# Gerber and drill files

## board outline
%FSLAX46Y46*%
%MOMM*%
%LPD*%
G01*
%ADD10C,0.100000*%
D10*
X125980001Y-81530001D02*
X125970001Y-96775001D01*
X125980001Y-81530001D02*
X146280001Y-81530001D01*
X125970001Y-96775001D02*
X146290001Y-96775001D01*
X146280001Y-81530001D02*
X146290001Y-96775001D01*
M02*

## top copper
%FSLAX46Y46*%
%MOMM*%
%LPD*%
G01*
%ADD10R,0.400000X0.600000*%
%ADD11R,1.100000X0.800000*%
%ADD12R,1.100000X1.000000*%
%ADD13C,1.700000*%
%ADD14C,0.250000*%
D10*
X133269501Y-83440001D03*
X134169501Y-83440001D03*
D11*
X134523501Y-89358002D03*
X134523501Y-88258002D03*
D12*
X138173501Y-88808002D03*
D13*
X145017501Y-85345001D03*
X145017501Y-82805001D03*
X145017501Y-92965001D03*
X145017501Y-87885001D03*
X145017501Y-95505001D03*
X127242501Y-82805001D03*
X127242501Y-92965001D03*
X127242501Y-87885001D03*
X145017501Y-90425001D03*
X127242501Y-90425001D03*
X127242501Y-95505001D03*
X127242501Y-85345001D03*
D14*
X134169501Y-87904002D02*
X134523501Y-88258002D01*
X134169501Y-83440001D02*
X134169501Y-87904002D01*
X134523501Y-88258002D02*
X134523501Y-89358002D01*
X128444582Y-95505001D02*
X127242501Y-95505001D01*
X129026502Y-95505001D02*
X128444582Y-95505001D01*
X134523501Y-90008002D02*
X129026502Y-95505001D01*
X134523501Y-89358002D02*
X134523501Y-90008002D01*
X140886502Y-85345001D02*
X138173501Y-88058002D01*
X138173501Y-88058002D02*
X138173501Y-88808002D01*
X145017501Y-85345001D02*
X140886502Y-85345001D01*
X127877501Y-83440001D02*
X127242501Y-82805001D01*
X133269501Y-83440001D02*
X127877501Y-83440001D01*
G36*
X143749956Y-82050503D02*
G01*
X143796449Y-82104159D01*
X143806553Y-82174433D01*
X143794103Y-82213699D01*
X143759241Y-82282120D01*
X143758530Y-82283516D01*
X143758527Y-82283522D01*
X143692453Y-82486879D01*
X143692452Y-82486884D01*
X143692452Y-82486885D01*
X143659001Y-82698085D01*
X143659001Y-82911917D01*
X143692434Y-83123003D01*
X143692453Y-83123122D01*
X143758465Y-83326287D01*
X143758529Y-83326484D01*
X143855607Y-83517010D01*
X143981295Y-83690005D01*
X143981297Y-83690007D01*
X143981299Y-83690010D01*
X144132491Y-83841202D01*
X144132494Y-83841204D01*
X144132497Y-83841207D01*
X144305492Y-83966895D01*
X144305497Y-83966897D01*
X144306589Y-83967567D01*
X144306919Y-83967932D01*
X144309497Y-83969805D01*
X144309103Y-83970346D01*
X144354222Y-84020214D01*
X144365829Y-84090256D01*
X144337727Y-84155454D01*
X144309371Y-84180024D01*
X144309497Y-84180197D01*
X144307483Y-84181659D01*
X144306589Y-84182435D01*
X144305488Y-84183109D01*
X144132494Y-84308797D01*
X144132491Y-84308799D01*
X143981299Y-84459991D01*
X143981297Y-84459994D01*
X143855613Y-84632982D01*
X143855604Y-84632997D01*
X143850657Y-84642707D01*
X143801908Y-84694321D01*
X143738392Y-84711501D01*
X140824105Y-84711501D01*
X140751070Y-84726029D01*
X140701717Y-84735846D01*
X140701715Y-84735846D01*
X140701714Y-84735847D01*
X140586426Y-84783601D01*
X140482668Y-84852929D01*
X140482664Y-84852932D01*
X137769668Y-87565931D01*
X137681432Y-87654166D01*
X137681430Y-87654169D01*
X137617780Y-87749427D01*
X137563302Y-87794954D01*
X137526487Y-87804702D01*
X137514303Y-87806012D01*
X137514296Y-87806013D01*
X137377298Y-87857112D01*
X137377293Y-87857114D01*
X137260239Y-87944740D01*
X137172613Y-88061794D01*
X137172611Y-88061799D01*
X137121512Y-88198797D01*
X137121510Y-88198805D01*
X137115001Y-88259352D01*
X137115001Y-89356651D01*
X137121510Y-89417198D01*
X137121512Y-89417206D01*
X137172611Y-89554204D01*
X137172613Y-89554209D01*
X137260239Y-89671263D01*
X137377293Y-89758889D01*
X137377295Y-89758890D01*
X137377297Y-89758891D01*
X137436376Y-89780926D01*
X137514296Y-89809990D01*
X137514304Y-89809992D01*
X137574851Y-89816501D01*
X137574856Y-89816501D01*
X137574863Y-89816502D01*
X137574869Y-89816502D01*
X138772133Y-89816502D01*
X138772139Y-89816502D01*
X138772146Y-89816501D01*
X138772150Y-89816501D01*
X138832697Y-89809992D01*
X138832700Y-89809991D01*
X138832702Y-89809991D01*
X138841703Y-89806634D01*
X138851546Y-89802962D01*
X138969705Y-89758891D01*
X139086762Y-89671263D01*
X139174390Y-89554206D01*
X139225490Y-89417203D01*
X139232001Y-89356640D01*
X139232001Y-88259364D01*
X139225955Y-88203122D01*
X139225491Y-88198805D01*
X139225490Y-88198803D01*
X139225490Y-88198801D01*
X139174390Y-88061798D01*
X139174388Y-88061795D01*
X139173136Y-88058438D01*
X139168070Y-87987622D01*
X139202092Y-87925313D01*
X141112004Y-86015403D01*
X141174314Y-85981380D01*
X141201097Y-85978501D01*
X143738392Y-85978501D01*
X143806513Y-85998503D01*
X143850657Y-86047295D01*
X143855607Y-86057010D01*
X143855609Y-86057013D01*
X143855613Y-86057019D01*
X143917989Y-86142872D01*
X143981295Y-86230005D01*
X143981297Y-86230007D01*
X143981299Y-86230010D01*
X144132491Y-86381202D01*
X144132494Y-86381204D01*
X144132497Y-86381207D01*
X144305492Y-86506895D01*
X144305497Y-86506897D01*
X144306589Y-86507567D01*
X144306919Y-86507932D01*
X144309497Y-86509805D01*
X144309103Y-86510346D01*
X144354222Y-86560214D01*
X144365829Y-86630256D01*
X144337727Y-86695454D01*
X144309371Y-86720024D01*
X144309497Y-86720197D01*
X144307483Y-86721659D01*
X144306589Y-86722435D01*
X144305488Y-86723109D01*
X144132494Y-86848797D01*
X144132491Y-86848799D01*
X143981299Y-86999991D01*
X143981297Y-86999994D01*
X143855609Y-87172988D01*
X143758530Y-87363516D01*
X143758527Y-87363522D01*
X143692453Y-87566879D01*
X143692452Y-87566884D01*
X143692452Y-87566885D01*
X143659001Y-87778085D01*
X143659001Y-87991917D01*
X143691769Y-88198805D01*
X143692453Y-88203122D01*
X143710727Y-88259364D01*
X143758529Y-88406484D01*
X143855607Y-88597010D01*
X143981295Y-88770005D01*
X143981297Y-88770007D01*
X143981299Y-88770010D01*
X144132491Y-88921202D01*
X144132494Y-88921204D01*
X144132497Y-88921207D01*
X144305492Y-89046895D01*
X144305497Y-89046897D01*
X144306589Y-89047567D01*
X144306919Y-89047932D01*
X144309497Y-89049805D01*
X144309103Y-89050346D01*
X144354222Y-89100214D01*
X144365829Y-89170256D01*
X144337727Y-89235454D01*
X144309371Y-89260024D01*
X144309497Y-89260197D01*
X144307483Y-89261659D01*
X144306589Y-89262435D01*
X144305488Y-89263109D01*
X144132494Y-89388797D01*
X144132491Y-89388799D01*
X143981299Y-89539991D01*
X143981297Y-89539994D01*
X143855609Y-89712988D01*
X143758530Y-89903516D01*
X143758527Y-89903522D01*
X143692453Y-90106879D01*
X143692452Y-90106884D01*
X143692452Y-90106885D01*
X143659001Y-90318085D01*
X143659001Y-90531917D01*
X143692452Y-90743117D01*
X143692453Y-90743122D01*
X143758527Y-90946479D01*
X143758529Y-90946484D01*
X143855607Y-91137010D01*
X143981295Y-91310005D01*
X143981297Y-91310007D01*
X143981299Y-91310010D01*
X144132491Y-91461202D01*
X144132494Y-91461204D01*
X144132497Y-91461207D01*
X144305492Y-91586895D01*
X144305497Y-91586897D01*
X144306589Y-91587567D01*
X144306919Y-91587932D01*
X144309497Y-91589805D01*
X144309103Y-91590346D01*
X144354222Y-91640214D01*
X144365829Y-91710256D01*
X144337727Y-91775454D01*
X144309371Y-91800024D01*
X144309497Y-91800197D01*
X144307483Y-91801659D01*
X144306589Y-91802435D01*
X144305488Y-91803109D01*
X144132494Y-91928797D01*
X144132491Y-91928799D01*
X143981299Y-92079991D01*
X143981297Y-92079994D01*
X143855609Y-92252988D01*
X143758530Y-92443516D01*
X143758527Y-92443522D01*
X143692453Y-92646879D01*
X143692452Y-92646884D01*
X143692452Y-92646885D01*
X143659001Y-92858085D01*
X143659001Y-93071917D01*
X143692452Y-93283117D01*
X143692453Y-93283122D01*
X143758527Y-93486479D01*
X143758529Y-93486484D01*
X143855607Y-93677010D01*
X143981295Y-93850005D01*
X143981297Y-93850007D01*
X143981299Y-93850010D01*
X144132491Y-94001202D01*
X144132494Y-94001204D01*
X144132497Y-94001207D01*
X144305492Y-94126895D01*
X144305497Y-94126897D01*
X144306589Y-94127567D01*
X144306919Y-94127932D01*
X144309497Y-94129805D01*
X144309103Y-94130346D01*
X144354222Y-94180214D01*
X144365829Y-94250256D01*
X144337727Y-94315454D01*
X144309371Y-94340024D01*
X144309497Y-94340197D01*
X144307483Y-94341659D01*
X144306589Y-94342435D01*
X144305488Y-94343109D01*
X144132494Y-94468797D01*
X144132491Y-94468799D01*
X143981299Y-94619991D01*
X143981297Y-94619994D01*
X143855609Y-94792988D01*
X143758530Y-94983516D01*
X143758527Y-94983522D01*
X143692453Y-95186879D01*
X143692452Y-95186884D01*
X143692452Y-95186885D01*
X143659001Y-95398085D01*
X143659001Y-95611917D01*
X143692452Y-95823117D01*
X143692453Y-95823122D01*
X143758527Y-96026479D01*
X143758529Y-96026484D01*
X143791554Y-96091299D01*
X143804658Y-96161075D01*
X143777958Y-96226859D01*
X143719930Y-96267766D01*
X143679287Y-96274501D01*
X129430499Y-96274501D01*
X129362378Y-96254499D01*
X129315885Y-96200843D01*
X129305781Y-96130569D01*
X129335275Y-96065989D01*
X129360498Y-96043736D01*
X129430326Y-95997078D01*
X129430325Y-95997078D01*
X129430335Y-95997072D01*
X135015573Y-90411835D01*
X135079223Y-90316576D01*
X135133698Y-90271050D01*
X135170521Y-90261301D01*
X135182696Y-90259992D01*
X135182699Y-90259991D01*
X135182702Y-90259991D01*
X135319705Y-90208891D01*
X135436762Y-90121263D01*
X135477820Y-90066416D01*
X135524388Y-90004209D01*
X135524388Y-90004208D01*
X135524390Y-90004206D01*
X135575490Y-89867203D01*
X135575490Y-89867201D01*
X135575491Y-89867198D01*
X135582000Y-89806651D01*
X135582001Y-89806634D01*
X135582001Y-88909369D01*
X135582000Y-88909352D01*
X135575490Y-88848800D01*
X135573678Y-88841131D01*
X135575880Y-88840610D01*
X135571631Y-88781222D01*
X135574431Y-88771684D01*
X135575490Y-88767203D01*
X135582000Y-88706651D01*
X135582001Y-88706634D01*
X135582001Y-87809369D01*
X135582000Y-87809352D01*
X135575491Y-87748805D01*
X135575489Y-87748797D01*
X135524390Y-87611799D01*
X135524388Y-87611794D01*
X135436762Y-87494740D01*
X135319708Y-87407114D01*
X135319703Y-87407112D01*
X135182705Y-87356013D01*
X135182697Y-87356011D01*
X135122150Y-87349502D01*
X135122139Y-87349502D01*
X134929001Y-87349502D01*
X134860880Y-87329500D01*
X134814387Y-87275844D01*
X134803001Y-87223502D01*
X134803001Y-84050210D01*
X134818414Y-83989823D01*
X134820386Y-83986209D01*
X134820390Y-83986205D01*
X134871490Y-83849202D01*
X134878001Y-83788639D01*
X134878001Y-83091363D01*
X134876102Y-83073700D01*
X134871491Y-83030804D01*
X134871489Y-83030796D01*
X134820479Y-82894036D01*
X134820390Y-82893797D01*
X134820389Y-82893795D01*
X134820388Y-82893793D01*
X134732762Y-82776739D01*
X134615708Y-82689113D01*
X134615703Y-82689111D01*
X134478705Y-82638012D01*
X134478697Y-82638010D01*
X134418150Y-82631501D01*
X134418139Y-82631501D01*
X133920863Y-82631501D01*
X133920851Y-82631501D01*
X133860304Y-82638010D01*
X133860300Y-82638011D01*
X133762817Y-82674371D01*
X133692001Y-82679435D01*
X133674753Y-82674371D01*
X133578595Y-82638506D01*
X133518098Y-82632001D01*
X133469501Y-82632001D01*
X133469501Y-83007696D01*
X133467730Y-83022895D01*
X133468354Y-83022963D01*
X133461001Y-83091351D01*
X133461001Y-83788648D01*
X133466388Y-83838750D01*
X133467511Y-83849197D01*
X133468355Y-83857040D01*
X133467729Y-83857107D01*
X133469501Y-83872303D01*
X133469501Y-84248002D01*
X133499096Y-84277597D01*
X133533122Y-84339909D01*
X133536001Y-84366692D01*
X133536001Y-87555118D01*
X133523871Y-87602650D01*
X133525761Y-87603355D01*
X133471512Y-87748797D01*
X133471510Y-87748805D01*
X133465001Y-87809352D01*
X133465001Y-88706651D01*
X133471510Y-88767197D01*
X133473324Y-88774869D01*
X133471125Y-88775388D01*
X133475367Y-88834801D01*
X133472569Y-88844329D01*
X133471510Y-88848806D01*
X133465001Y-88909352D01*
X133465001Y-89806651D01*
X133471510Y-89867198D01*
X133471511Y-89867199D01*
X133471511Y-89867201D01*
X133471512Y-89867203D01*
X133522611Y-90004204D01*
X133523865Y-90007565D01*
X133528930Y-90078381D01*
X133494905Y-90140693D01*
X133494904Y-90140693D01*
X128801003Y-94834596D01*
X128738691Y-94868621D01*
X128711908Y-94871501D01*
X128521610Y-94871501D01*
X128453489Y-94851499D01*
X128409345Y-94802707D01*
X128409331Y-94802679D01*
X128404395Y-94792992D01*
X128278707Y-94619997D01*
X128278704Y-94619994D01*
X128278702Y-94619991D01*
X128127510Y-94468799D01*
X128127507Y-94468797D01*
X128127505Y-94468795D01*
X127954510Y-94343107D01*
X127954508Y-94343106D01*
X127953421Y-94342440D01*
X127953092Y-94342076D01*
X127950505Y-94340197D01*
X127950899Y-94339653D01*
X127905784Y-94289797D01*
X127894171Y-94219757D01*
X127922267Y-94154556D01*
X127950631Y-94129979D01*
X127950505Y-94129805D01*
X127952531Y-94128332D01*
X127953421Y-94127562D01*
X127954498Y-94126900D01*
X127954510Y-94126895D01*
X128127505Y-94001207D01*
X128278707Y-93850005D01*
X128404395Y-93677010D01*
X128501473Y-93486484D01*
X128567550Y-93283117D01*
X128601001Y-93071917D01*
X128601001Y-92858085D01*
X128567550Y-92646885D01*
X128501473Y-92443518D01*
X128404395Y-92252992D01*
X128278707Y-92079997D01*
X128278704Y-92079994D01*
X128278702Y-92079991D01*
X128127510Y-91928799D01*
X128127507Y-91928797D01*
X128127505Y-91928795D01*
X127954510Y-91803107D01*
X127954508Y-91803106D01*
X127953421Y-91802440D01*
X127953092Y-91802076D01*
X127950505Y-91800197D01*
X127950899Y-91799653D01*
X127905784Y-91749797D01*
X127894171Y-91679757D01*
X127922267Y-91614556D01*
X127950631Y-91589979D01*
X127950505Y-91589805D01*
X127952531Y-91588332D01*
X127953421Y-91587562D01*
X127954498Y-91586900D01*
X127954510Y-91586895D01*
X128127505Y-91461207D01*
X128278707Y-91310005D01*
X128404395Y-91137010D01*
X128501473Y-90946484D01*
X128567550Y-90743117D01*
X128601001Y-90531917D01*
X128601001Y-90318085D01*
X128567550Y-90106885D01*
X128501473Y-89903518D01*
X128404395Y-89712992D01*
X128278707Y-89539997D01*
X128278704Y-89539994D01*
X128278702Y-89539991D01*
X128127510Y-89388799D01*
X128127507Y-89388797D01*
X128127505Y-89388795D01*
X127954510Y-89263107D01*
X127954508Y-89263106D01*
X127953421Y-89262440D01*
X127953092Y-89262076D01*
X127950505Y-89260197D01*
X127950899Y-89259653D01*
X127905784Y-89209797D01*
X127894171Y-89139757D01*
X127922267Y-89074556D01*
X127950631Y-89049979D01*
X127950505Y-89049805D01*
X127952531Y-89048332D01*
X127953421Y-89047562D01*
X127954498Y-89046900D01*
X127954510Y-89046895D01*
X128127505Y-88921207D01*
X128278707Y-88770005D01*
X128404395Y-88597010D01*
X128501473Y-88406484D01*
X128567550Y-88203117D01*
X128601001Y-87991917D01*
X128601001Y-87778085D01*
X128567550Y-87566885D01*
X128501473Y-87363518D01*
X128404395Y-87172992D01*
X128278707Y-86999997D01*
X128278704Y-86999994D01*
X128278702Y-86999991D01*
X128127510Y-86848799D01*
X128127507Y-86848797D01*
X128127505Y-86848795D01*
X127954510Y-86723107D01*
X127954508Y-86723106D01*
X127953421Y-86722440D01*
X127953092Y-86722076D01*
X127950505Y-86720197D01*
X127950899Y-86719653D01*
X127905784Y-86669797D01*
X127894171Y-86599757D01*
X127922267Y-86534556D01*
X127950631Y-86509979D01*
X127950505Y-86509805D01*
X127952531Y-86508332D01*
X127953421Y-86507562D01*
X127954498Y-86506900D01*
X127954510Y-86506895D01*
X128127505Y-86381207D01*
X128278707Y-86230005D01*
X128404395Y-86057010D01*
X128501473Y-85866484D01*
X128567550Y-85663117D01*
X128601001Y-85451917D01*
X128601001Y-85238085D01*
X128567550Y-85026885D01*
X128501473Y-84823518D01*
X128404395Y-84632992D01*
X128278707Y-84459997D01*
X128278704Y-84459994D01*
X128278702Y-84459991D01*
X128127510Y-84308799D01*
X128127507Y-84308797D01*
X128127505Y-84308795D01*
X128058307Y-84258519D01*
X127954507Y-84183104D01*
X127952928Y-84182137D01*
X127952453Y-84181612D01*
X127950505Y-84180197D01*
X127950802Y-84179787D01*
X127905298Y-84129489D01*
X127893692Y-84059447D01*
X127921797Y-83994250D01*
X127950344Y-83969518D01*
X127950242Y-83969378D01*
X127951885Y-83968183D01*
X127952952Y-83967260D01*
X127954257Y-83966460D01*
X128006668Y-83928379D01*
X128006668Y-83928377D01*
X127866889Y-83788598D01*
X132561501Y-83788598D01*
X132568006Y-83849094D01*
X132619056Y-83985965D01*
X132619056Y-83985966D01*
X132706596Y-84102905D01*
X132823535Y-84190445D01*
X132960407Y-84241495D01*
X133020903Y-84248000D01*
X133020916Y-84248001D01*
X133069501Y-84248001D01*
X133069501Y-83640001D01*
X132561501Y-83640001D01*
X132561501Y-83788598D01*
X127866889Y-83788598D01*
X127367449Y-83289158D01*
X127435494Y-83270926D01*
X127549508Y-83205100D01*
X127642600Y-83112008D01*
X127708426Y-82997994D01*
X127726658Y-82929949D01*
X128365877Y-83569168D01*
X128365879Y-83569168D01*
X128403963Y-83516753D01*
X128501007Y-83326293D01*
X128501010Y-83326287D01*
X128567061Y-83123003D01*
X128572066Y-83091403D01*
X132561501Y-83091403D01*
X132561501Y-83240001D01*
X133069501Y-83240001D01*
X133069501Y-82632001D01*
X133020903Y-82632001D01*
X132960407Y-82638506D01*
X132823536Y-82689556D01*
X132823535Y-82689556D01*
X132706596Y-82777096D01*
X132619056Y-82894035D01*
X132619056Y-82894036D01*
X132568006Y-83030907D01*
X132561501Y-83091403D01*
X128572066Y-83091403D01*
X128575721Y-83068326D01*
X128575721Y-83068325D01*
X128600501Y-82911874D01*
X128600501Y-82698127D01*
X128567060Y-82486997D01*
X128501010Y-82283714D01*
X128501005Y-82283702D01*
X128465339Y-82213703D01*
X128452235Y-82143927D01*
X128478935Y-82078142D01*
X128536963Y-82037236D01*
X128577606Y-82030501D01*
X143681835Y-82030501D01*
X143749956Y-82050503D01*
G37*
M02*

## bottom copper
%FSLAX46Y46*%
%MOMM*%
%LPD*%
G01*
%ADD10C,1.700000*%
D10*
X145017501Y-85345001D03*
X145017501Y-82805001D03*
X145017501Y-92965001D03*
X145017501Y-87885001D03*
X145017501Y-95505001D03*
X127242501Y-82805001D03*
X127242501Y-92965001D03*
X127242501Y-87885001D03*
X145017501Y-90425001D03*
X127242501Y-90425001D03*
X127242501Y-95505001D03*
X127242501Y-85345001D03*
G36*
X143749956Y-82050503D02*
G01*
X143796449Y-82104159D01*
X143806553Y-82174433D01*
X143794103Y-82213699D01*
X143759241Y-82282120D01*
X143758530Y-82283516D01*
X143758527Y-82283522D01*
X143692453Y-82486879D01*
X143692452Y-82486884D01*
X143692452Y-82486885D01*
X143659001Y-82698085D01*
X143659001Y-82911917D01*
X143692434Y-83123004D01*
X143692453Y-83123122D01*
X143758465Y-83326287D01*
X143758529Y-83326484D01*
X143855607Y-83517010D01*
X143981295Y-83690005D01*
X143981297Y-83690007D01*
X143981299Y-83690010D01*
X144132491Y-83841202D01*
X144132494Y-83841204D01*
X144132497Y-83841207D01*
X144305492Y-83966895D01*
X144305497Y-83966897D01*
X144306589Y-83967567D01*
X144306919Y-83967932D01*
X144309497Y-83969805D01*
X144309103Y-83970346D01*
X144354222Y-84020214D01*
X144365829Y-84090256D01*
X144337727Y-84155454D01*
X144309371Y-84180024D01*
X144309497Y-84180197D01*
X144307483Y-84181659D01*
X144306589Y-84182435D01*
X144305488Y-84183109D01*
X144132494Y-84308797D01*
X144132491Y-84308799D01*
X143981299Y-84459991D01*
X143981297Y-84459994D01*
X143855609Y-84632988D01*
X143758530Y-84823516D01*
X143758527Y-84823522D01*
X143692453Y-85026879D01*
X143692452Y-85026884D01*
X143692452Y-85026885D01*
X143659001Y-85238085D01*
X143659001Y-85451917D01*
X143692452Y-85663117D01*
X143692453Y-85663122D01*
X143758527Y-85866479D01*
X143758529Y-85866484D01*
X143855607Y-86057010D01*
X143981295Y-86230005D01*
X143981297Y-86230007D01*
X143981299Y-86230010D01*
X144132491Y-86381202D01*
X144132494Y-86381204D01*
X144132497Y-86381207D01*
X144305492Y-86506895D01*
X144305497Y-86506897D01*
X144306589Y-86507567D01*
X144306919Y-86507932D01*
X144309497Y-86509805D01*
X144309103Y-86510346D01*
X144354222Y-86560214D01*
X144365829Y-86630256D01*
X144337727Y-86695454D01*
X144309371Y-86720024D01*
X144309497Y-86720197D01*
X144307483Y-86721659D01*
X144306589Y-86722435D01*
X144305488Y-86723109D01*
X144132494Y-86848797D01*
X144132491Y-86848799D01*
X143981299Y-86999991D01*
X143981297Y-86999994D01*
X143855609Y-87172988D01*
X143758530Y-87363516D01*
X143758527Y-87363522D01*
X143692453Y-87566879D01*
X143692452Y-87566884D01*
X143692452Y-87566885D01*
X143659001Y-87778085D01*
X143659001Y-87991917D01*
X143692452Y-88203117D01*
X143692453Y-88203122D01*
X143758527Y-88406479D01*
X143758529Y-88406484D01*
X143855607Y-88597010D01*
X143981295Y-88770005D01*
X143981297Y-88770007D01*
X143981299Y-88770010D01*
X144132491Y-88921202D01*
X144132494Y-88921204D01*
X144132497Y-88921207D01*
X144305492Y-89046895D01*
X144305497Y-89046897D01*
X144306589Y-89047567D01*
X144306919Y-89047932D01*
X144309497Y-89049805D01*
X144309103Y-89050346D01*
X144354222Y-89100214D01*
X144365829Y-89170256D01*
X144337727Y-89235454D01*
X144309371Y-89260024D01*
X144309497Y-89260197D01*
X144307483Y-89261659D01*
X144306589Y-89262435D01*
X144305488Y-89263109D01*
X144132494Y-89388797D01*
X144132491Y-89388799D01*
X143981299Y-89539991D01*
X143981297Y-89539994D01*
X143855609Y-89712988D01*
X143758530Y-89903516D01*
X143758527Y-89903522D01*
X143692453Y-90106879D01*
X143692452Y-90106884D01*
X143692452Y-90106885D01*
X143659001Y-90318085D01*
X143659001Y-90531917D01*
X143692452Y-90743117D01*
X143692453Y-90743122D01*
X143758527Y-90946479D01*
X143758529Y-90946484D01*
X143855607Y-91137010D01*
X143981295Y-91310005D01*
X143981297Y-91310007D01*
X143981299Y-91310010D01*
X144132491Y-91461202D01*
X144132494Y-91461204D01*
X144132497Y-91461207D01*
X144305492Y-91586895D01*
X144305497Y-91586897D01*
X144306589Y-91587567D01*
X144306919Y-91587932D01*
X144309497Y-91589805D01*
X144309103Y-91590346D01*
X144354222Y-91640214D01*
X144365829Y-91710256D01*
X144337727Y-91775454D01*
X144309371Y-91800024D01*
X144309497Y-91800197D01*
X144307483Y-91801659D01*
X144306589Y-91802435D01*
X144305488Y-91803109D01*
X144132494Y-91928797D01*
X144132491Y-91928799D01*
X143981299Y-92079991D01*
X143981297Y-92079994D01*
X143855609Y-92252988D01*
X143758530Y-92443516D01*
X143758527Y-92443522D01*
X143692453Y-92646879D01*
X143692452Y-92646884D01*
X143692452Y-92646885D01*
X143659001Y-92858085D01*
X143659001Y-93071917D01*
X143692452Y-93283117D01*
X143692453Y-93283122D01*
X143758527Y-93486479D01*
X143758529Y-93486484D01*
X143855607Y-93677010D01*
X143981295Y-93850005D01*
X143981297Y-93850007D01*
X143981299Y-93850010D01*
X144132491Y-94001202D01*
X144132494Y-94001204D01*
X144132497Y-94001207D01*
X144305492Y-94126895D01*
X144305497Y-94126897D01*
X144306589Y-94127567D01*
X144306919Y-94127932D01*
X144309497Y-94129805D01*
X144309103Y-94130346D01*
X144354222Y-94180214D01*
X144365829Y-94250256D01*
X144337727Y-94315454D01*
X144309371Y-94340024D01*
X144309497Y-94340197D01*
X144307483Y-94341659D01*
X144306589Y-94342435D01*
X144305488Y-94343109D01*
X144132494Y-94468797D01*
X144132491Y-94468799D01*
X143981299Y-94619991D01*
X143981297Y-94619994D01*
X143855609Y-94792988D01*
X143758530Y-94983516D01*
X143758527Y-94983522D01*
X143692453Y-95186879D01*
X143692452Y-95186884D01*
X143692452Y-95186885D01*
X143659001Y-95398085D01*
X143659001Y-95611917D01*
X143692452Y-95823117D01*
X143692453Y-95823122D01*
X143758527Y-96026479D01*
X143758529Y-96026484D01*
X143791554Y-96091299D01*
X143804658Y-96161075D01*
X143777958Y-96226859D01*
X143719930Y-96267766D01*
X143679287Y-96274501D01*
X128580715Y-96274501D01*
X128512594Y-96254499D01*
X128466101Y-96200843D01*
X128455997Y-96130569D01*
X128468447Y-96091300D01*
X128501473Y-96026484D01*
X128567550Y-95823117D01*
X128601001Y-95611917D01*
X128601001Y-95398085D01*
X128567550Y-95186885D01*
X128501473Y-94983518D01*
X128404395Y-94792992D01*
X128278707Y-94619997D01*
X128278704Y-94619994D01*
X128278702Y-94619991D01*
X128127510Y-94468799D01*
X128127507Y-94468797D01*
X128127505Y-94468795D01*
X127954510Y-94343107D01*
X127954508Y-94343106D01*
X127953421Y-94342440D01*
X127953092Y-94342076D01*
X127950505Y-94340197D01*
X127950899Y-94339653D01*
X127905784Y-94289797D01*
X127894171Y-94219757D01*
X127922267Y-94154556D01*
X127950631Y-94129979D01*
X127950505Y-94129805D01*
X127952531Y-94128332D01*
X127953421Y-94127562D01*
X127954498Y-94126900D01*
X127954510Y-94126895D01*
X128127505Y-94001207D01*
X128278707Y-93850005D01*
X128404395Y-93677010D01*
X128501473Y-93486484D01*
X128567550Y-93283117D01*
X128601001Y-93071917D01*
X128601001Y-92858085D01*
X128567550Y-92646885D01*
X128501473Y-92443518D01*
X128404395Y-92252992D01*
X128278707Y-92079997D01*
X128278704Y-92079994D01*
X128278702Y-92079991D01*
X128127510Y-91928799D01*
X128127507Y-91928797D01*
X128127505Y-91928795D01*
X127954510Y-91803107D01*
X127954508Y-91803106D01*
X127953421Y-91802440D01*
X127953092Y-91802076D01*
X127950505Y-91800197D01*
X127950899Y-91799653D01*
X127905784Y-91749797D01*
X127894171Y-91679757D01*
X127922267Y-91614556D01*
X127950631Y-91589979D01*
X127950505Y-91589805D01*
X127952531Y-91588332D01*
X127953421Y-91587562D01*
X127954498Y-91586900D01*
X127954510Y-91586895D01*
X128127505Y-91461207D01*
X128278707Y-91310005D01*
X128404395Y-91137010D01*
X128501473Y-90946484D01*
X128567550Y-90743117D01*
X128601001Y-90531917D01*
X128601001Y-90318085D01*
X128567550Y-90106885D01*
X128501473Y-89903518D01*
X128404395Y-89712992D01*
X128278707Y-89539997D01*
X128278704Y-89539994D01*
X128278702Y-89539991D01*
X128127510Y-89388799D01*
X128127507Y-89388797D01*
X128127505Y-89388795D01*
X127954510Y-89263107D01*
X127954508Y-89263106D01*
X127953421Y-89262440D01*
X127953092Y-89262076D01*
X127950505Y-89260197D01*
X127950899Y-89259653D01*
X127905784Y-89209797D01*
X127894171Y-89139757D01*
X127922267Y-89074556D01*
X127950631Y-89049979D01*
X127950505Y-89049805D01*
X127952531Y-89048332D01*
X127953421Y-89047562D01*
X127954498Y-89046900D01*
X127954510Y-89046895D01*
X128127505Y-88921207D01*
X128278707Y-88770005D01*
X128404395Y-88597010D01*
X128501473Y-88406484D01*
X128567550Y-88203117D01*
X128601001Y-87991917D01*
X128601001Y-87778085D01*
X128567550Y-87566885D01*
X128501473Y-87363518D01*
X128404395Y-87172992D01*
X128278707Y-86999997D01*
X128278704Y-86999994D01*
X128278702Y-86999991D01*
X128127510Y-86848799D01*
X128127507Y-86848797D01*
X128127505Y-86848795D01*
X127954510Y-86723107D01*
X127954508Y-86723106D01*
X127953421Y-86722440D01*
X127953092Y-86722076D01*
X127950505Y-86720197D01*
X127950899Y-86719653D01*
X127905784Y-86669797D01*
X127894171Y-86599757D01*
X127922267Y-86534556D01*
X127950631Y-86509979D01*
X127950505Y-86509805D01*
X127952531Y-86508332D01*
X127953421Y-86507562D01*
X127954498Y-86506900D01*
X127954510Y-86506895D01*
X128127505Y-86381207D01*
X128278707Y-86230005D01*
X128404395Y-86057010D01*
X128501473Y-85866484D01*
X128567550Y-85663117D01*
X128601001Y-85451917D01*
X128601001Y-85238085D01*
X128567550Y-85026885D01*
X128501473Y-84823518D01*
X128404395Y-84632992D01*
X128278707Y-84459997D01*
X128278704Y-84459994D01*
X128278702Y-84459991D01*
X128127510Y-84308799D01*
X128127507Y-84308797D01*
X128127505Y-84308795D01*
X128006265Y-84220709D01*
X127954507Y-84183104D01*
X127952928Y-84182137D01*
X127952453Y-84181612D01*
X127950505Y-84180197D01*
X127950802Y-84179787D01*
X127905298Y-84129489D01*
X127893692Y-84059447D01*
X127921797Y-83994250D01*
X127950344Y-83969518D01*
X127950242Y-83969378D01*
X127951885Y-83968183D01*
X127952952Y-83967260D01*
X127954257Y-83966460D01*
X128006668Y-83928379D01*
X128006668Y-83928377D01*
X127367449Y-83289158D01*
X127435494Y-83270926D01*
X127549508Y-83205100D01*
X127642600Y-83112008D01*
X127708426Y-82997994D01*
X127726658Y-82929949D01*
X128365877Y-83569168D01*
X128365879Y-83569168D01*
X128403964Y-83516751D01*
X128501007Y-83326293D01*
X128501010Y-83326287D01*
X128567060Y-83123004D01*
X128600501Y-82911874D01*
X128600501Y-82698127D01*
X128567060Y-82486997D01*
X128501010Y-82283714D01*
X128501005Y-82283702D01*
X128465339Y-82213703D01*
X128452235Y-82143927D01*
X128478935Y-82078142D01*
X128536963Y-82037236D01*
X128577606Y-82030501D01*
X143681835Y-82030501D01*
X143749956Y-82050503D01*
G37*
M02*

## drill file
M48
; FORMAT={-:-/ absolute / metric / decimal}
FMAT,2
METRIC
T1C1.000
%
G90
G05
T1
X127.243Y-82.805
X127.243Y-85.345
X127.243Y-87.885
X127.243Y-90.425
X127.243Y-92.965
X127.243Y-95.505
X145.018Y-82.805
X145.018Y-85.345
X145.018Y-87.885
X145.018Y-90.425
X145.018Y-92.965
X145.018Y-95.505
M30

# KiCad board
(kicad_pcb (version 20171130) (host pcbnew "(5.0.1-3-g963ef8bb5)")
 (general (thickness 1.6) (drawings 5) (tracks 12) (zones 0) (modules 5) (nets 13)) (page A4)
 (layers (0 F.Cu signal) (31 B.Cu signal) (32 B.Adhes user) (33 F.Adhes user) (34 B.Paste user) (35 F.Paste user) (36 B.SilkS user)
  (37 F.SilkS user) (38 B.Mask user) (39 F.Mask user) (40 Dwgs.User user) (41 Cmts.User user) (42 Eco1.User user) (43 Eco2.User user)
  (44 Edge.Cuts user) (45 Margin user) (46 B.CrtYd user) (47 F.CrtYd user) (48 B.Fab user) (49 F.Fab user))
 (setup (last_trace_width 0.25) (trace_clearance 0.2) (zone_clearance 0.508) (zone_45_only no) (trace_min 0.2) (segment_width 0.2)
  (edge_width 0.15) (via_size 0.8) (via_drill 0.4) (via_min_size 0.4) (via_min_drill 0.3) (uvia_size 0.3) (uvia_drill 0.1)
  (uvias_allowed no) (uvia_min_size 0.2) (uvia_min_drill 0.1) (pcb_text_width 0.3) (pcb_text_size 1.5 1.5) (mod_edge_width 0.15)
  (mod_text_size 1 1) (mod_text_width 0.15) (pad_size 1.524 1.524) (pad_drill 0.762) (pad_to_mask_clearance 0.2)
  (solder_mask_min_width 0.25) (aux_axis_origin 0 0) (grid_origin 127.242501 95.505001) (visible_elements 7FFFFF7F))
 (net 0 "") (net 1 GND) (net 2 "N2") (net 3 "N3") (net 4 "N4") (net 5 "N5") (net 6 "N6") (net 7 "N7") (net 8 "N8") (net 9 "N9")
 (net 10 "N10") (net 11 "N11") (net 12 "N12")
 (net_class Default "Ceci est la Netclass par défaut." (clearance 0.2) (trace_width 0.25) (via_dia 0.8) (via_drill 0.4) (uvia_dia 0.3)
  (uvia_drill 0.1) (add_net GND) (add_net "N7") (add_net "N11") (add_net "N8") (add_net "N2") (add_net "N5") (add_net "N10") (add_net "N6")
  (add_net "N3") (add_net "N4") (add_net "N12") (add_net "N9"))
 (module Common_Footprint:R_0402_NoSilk (layer F.Cu) (at 133.719501 83.440001 180)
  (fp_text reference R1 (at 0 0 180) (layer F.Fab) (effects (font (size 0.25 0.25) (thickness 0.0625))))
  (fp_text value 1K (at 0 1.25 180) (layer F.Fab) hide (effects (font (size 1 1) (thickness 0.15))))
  (pad 2 smd rect (at 0.45 0 180) (size 0.4 0.6) (layers F.Cu F.Paste F.Mask) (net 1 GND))
  (pad 1 smd rect (at -0.45 0 180) (size 0.4 0.6) (layers F.Cu F.Paste F.Mask) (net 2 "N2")))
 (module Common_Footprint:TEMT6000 (layer F.Cu) (at 136.348501 88.808002)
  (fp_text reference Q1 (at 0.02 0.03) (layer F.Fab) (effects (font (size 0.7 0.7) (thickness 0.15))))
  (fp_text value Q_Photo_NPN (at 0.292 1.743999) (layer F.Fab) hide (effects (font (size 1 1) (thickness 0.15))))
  (pad 2 smd rect (at -1.825 0.55) (size 1.1 0.8) (layers F.Cu F.Paste F.Mask) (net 2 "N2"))
  (pad 2 smd rect (at -1.825 -0.55) (size 1.1 0.8) (layers F.Cu F.Paste F.Mask) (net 2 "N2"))
  (pad 1 smd rect (at 1.825 0) (size 1.1 1) (layers F.Cu F.Paste F.Mask) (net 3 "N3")))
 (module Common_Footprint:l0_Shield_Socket (layer F.Cu) (at 136.130001 89.155001)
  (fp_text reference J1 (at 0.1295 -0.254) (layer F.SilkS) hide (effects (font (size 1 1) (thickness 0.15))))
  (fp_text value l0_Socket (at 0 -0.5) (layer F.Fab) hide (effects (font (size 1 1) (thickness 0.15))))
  (fp_line (start -10.15 -7.625) (end -10.16 7.62) (layer Edge.Cuts) (width 0.1))
  (fp_line (start -10.15 -7.625) (end 10.15 -7.625) (layer Edge.Cuts) (width 0.1))
  (fp_line (start -10.16 7.62) (end 10.16 7.62) (layer Edge.Cuts) (width 0.1))
  (fp_line (start 10.15 -7.625) (end 10.16 7.62) (layer Edge.Cuts) (width 0.1))
  (pad 5 thru_hole circle (at 8.8875 -3.81 270) (size 1.7 1.7) (drill 1) (layers *.Cu *.Mask) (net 3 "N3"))
  (pad 6 thru_hole circle (at 8.8875 -6.35 270) (size 1.7 1.7) (drill 1) (layers *.Cu *.Mask) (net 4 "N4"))
  (pad 2 thru_hole circle (at 8.8875 3.81 270) (size 1.7 1.7) (drill 1) (layers *.Cu *.Mask) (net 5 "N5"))
  (pad 4 thru_hole circle (at 8.8875 -1.27 270) (size 1.7 1.7) (drill 1) (layers *.Cu *.Mask) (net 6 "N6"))
  (pad 1 thru_hole circle (at 8.8875 6.35 270) (size 1.7 1.7) (drill 1) (layers *.Cu *.Mask) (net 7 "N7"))
  (pad 7 thru_hole circle (at -8.8875 -6.35 270) (size 1.7 1.7) (drill 1) (layers *.Cu *.Mask) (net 1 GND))
  (pad 11 thru_hole circle (at -8.8875 3.81 270) (size 1.7 1.7) (drill 1) (layers *.Cu *.Mask) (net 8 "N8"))
  (pad 9 thru_hole circle (at -8.8875 -1.27 270) (size 1.7 1.7) (drill 1) (layers *.Cu *.Mask) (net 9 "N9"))
  (pad 3 thru_hole circle (at 8.8875 1.27 270) (size 1.7 1.7) (drill 1) (layers *.Cu *.Mask) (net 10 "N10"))
  (pad 10 thru_hole circle (at -8.8875 1.27 270) (size 1.7 1.7) (drill 1) (layers *.Cu *.Mask) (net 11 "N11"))
  (pad 12 thru_hole circle (at -8.8875 6.35 270) (size 1.7 1.7) (drill 1) (layers *.Cu *.Mask) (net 2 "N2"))
  (pad 8 thru_hole circle (at -8.8875 -3.81 270) (size 1.7 1.7) (drill 1) (layers *.Cu *.Mask) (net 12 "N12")))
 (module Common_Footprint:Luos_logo (layer F.Cu) (at 136.640501 92.330001)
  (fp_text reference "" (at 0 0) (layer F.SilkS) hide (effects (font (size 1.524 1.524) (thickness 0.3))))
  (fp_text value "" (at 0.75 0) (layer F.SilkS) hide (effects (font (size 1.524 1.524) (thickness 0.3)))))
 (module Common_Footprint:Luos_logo (layer B.Cu) (at 136.767501 88.393001)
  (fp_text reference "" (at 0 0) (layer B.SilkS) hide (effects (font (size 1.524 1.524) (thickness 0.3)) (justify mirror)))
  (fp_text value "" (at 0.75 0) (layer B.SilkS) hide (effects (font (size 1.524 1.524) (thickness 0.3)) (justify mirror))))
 (segment (start 134.169501 87.904002) (end 134.523501 88.258002) (width 0.25) (layer F.Cu) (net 2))
 (segment (start 134.169501 83.440001) (end 134.169501 87.904002) (width 0.25) (layer F.Cu) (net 2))
 (segment (start 134.523501 88.258002) (end 134.523501 89.358002) (width 0.25) (layer F.Cu) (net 2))
 (segment (start 128.444582 95.505001) (end 127.242501 95.505001) (width 0.25) (layer F.Cu) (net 2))
 (segment (start 129.026502 95.505001) (end 128.444582 95.505001) (width 0.25) (layer F.Cu) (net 2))
 (segment (start 134.523501 90.008002) (end 129.026502 95.505001) (width 0.25) (layer F.Cu) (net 2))
 (segment (start 134.523501 89.358002) (end 134.523501 90.008002) (width 0.25) (layer F.Cu) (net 2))
 (segment (start 140.886502 85.345001) (end 138.173501 88.058002) (width 0.25) (layer F.Cu) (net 3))
 (segment (start 138.173501 88.058002) (end 138.173501 88.808002) (width 0.25) (layer F.Cu) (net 3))
 (segment (start 145.017501 85.345001) (end 140.886502 85.345001) (width 0.25) (layer F.Cu) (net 3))
 (segment (start 127.877501 83.440001) (end 127.242501 82.805001) (width 0.25) (layer F.Cu) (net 1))
 (segment (start 133.269501 83.440001) (end 127.877501 83.440001) (width 0.25) (layer F.Cu) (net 1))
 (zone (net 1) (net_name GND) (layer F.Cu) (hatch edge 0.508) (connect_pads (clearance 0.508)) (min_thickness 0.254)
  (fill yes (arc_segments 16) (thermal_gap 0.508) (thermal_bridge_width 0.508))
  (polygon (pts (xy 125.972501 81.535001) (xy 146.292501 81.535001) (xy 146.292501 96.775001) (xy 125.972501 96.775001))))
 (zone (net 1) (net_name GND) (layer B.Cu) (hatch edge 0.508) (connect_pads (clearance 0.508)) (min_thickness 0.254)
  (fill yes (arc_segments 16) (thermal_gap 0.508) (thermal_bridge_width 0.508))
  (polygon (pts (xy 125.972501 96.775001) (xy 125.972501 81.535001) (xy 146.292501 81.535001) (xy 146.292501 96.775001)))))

